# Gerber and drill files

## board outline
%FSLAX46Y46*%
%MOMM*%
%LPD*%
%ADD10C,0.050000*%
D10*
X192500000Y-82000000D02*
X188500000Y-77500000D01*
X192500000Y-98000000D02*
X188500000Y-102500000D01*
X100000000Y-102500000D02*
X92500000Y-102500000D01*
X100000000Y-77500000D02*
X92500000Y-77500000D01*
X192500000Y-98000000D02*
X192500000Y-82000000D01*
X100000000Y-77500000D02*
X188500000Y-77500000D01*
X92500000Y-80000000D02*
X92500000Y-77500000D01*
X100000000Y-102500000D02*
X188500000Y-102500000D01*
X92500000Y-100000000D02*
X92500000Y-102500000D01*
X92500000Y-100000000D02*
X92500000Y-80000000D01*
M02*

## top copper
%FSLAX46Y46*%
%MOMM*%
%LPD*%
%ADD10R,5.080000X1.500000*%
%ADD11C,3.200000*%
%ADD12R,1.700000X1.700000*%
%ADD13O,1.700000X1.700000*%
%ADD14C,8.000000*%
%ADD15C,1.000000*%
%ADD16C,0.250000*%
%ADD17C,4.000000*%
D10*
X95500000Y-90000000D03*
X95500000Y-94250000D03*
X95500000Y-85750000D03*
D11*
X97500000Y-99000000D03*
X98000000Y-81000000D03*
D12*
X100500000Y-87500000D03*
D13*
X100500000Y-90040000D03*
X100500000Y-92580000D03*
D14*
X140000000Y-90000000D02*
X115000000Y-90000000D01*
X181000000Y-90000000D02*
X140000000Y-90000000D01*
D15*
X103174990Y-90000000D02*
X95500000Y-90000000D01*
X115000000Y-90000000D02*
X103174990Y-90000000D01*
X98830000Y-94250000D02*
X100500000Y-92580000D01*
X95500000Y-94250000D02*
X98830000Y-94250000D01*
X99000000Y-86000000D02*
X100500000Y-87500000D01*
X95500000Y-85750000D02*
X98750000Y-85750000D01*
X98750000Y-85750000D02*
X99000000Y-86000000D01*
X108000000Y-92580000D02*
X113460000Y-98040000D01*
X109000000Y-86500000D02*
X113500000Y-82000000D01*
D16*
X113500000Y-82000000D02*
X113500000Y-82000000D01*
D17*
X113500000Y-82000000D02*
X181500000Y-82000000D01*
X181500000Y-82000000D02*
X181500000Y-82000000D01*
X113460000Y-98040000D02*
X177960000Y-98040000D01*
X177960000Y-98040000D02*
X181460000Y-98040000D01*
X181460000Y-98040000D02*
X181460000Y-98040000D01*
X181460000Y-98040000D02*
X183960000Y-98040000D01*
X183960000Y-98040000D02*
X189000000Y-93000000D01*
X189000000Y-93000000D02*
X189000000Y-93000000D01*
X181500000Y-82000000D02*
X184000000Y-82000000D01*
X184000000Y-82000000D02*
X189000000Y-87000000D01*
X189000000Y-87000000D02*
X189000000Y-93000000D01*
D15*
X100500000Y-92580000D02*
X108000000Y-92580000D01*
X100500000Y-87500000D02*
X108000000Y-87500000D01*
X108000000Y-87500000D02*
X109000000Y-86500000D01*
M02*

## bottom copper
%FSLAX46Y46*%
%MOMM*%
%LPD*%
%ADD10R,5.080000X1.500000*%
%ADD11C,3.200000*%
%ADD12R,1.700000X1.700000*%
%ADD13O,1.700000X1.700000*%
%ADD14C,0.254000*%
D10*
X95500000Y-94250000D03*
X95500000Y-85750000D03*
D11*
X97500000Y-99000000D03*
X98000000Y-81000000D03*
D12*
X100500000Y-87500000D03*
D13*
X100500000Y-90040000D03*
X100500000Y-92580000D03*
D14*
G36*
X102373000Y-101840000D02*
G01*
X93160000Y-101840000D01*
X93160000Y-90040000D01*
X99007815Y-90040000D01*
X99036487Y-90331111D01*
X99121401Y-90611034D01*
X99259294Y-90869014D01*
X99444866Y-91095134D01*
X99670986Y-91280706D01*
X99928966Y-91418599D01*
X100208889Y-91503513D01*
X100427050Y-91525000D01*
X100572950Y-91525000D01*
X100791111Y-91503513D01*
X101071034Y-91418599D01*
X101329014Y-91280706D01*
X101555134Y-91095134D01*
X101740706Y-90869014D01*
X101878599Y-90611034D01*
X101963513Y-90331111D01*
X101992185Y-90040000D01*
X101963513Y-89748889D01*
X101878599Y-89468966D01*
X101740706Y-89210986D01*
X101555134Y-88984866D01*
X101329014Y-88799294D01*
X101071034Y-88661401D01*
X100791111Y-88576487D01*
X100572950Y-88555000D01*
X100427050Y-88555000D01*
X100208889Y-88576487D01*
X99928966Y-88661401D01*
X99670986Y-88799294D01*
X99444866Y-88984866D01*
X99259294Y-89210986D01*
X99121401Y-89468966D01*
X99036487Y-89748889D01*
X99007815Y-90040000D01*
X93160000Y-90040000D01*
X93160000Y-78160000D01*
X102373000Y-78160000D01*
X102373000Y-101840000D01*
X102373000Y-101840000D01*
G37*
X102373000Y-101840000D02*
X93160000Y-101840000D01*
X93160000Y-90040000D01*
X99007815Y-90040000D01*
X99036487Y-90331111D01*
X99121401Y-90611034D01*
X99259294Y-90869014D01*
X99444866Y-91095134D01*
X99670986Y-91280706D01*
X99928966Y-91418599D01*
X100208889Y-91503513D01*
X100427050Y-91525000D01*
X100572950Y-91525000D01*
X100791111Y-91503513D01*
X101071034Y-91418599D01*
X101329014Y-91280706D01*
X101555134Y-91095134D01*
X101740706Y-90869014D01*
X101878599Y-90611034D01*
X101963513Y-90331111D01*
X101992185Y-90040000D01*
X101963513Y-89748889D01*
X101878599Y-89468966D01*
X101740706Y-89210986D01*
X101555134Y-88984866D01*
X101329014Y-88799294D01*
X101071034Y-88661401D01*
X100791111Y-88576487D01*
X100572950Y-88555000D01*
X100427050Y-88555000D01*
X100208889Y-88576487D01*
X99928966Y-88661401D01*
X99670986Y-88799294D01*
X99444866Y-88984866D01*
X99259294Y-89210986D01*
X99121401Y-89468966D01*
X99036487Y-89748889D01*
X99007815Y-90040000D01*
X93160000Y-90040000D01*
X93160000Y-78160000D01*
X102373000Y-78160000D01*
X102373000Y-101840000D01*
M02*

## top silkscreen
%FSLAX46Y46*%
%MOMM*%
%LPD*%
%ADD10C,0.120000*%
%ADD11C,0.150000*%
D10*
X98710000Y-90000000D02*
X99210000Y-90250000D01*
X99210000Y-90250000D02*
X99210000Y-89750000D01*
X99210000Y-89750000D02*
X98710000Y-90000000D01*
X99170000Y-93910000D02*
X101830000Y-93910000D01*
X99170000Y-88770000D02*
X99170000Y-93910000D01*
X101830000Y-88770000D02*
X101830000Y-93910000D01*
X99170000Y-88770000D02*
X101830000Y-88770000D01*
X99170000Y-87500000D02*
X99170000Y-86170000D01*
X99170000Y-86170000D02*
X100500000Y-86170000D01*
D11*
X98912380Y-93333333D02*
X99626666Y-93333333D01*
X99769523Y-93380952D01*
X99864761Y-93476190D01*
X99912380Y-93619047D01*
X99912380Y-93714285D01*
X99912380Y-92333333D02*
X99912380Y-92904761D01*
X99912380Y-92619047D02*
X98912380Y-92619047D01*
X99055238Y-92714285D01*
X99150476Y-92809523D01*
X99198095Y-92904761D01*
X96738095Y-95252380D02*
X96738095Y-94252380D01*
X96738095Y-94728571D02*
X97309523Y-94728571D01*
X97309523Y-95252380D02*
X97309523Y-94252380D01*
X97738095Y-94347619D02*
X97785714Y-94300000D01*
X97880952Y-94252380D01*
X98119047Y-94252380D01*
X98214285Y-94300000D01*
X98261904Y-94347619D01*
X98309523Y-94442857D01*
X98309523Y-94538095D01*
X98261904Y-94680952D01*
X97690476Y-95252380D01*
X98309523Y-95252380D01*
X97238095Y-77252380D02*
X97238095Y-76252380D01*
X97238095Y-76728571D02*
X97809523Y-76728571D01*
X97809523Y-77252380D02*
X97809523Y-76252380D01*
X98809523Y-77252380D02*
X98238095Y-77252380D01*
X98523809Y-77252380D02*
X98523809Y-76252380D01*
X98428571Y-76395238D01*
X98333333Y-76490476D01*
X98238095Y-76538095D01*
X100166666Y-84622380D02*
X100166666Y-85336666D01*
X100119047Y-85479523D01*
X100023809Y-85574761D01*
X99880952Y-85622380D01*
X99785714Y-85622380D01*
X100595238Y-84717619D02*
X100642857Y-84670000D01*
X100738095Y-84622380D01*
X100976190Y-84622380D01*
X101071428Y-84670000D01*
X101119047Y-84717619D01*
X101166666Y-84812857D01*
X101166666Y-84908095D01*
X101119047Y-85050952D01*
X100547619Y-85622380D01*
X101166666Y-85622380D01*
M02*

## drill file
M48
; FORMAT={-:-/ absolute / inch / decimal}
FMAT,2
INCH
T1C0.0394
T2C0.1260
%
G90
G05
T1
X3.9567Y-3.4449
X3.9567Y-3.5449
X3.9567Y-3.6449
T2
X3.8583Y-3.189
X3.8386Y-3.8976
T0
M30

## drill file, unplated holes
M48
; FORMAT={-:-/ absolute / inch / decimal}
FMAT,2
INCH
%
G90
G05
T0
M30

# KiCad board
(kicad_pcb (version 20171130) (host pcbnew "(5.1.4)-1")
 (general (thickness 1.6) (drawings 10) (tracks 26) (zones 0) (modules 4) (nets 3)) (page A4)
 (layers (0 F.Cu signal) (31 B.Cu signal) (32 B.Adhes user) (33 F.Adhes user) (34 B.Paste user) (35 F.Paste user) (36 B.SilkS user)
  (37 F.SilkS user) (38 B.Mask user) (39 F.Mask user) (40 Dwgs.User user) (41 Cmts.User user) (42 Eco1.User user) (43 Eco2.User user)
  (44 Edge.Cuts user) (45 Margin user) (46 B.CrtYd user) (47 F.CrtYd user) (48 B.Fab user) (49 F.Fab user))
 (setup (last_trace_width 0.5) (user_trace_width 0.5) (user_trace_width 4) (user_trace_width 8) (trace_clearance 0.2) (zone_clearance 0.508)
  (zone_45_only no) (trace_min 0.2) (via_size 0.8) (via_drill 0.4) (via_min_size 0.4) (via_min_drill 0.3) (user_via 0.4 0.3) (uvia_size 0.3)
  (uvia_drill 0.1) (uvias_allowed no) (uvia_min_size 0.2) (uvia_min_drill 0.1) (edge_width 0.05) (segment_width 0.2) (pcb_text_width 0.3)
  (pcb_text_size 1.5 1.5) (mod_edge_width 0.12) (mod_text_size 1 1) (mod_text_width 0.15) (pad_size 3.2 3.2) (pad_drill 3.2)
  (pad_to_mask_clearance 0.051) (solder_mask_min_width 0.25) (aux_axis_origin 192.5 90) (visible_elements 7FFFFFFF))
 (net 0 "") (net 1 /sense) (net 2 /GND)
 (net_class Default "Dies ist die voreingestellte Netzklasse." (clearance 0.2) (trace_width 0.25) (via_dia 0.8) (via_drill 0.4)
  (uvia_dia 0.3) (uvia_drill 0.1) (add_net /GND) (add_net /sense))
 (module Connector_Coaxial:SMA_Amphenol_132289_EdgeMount (layer F.Cu) (at 95.5 90 180)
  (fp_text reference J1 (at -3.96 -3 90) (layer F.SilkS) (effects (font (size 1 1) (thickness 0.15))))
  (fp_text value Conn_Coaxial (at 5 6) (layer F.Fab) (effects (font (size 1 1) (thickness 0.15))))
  (fp_line (start -3.21 0) (end -3.71 -0.25) (layer F.SilkS) (width 0.12))
  (fp_line (start -3.71 -0.25) (end -3.71 0.25) (layer F.SilkS) (width 0.12))
  (fp_line (start -3.71 0.25) (end -3.21 0) (layer F.SilkS) (width 0.12))
  (pad 1 smd rect (at 0 0 270) (size 1.5 5.08) (layers F.Cu F.Paste F.Mask) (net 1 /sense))
  (pad 2 smd rect (at 0 -4.25 270) (size 1.5 5.08) (layers F.Cu F.Paste F.Mask) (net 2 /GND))
  (pad 2 smd rect (at 0 4.25 270) (size 1.5 5.08) (layers F.Cu F.Paste F.Mask) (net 2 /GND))
  (pad 2 smd rect (at 0 -4.25 270) (size 1.5 5.08) (layers B.Cu B.Paste B.Mask) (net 2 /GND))
  (pad 2 smd rect (at 0 4.25 270) (size 1.5 5.08) (layers B.Cu B.Paste B.Mask) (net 2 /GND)))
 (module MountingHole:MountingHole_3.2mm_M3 (layer F.Cu) (at 97.5 99)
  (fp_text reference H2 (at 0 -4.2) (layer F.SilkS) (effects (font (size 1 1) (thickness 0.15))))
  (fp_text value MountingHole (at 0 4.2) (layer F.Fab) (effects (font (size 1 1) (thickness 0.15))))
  (pad 1 thru_hole circle (at 0 0) (size 3.2 3.2) (drill 3.2) (layers *.Cu *.Mask) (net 2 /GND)))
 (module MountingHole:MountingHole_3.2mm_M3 (layer F.Cu) (at 98 81)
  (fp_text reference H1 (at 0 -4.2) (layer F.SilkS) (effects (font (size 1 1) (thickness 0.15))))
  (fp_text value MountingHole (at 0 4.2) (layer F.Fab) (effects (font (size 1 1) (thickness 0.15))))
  (pad 1 thru_hole circle (at 0 0) (size 3.2 3.2) (drill 3.2) (layers *.Cu *.Mask) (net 2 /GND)))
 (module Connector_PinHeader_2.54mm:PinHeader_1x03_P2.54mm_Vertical (layer F.Cu) (at 100.5 87.5)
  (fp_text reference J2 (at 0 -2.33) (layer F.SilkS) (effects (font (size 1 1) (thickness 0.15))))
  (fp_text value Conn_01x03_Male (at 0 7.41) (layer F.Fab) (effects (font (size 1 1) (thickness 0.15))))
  (fp_line (start -1.33 6.41) (end 1.33 6.41) (layer F.SilkS) (width 0.12))
  (fp_line (start -1.33 1.27) (end -1.33 6.41) (layer F.SilkS) (width 0.12))
  (fp_line (start 1.33 1.27) (end 1.33 6.41) (layer F.SilkS) (width 0.12))
  (fp_line (start -1.33 1.27) (end 1.33 1.27) (layer F.SilkS) (width 0.12))
  (fp_line (start -1.33 0) (end -1.33 -1.33) (layer F.SilkS) (width 0.12))
  (fp_line (start -1.33 -1.33) (end 0 -1.33) (layer F.SilkS) (width 0.12))
  (pad 1 thru_hole rect (at 0 0) (size 1.7 1.7) (drill 1) (layers *.Cu *.Mask) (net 2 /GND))
  (pad 2 thru_hole oval (at 0 2.54) (size 1.7 1.7) (drill 1) (layers *.Cu *.Mask) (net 1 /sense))
  (pad 3 thru_hole oval (at 0 5.08) (size 1.7 1.7) (drill 1) (layers *.Cu *.Mask) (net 2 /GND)))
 (gr_line (start 192.5 82) (end 188.5 77.5) (layer Edge.Cuts) (width 0.05))
 (gr_line (start 192.5 98) (end 188.5 102.5) (layer Edge.Cuts) (width 0.05))
 (gr_line (start 100 102.5) (end 92.5 102.5) (layer Edge.Cuts) (width 0.05))
 (gr_line (start 100 77.5) (end 92.5 77.5) (layer Edge.Cuts) (width 0.05))
 (gr_line (start 192.5 98) (end 192.5 82) (layer Edge.Cuts) (width 0.05))
 (gr_line (start 100 77.5) (end 188.5 77.5) (layer Edge.Cuts) (width 0.05))
 (gr_line (start 92.5 80) (end 92.5 77.5) (layer Edge.Cuts) (width 0.05))
 (gr_line (start 100 102.5) (end 188.5 102.5) (layer Edge.Cuts) (width 0.05))
 (gr_line (start 92.5 100) (end 92.5 102.5) (layer Edge.Cuts) (width 0.05))
 (gr_line (start 92.5 100) (end 92.5 80) (layer Edge.Cuts) (width 0.05))
 (segment (start 140 90) (end 115 90) (width 8) (layer F.Cu) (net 1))
 (segment (start 181 90) (end 140 90) (width 8) (layer F.Cu) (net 1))
 (segment (start 103.17499 90) (end 95.5 90) (width 1) (layer F.Cu) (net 1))
 (segment (start 115 90) (end 103.17499 90) (width 1) (layer F.Cu) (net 1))
 (segment (start 98.83 94.25) (end 100.5 92.58) (width 1) (layer F.Cu) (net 2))
 (segment (start 95.5 94.25) (end 98.83 94.25) (width 1) (layer F.Cu) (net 2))
 (segment (start 99 86) (end 100.5 87.5) (width 1) (layer F.Cu) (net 2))
 (segment (start 95.5 85.75) (end 98.75 85.75) (width 1) (layer F.Cu) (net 2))
 (segment (start 98.75 85.75) (end 99 86) (width 1) (layer F.Cu) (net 2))
 (segment (start 108 92.58) (end 113.46 98.04) (width 1) (layer F.Cu) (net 2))
 (segment (start 109 86.5) (end 113.5 82) (width 1) (layer F.Cu) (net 2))
 (segment (start 113.5 82) (end 113.5 82) (width 0.25) (layer F.Cu) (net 2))
 (segment (start 113.5 82) (end 181.5 82) (width 4) (layer F.Cu) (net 2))
 (segment (start 181.5 82) (end 181.5 82) (width 4) (layer F.Cu) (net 2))
 (segment (start 113.46 98.04) (end 177.96 98.04) (width 4) (layer F.Cu) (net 2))
 (segment (start 177.96 98.04) (end 181.46 98.04) (width 4) (layer F.Cu) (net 2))
 (segment (start 181.46 98.04) (end 181.46 98.04) (width 4) (layer F.Cu) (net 2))
 (segment (start 181.46 98.04) (end 183.96 98.04) (width 4) (layer F.Cu) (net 2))
 (segment (start 183.96 98.04) (end 189 93) (width 4) (layer F.Cu) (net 2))
 (segment (start 189 93) (end 189 93) (width 4) (layer F.Cu) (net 2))
 (segment (start 181.5 82) (end 184 82) (width 4) (layer F.Cu) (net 2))
 (segment (start 184 82) (end 189 87) (width 4) (layer F.Cu) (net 2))
 (segment (start 189 87) (end 189 93) (width 4) (layer F.Cu) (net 2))
 (segment (start 100.5 92.58) (end 108 92.58) (width 1) (layer F.Cu) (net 2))
 (segment (start 100.5 87.5) (end 108 87.5) (width 1) (layer F.Cu) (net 2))
 (segment (start 108 87.5) (end 109 86.5) (width 1) (layer F.Cu) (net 2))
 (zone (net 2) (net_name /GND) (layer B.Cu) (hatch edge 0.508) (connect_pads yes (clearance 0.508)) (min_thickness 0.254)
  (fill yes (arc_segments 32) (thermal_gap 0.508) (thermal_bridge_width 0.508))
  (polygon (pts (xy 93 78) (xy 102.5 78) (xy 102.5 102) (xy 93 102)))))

